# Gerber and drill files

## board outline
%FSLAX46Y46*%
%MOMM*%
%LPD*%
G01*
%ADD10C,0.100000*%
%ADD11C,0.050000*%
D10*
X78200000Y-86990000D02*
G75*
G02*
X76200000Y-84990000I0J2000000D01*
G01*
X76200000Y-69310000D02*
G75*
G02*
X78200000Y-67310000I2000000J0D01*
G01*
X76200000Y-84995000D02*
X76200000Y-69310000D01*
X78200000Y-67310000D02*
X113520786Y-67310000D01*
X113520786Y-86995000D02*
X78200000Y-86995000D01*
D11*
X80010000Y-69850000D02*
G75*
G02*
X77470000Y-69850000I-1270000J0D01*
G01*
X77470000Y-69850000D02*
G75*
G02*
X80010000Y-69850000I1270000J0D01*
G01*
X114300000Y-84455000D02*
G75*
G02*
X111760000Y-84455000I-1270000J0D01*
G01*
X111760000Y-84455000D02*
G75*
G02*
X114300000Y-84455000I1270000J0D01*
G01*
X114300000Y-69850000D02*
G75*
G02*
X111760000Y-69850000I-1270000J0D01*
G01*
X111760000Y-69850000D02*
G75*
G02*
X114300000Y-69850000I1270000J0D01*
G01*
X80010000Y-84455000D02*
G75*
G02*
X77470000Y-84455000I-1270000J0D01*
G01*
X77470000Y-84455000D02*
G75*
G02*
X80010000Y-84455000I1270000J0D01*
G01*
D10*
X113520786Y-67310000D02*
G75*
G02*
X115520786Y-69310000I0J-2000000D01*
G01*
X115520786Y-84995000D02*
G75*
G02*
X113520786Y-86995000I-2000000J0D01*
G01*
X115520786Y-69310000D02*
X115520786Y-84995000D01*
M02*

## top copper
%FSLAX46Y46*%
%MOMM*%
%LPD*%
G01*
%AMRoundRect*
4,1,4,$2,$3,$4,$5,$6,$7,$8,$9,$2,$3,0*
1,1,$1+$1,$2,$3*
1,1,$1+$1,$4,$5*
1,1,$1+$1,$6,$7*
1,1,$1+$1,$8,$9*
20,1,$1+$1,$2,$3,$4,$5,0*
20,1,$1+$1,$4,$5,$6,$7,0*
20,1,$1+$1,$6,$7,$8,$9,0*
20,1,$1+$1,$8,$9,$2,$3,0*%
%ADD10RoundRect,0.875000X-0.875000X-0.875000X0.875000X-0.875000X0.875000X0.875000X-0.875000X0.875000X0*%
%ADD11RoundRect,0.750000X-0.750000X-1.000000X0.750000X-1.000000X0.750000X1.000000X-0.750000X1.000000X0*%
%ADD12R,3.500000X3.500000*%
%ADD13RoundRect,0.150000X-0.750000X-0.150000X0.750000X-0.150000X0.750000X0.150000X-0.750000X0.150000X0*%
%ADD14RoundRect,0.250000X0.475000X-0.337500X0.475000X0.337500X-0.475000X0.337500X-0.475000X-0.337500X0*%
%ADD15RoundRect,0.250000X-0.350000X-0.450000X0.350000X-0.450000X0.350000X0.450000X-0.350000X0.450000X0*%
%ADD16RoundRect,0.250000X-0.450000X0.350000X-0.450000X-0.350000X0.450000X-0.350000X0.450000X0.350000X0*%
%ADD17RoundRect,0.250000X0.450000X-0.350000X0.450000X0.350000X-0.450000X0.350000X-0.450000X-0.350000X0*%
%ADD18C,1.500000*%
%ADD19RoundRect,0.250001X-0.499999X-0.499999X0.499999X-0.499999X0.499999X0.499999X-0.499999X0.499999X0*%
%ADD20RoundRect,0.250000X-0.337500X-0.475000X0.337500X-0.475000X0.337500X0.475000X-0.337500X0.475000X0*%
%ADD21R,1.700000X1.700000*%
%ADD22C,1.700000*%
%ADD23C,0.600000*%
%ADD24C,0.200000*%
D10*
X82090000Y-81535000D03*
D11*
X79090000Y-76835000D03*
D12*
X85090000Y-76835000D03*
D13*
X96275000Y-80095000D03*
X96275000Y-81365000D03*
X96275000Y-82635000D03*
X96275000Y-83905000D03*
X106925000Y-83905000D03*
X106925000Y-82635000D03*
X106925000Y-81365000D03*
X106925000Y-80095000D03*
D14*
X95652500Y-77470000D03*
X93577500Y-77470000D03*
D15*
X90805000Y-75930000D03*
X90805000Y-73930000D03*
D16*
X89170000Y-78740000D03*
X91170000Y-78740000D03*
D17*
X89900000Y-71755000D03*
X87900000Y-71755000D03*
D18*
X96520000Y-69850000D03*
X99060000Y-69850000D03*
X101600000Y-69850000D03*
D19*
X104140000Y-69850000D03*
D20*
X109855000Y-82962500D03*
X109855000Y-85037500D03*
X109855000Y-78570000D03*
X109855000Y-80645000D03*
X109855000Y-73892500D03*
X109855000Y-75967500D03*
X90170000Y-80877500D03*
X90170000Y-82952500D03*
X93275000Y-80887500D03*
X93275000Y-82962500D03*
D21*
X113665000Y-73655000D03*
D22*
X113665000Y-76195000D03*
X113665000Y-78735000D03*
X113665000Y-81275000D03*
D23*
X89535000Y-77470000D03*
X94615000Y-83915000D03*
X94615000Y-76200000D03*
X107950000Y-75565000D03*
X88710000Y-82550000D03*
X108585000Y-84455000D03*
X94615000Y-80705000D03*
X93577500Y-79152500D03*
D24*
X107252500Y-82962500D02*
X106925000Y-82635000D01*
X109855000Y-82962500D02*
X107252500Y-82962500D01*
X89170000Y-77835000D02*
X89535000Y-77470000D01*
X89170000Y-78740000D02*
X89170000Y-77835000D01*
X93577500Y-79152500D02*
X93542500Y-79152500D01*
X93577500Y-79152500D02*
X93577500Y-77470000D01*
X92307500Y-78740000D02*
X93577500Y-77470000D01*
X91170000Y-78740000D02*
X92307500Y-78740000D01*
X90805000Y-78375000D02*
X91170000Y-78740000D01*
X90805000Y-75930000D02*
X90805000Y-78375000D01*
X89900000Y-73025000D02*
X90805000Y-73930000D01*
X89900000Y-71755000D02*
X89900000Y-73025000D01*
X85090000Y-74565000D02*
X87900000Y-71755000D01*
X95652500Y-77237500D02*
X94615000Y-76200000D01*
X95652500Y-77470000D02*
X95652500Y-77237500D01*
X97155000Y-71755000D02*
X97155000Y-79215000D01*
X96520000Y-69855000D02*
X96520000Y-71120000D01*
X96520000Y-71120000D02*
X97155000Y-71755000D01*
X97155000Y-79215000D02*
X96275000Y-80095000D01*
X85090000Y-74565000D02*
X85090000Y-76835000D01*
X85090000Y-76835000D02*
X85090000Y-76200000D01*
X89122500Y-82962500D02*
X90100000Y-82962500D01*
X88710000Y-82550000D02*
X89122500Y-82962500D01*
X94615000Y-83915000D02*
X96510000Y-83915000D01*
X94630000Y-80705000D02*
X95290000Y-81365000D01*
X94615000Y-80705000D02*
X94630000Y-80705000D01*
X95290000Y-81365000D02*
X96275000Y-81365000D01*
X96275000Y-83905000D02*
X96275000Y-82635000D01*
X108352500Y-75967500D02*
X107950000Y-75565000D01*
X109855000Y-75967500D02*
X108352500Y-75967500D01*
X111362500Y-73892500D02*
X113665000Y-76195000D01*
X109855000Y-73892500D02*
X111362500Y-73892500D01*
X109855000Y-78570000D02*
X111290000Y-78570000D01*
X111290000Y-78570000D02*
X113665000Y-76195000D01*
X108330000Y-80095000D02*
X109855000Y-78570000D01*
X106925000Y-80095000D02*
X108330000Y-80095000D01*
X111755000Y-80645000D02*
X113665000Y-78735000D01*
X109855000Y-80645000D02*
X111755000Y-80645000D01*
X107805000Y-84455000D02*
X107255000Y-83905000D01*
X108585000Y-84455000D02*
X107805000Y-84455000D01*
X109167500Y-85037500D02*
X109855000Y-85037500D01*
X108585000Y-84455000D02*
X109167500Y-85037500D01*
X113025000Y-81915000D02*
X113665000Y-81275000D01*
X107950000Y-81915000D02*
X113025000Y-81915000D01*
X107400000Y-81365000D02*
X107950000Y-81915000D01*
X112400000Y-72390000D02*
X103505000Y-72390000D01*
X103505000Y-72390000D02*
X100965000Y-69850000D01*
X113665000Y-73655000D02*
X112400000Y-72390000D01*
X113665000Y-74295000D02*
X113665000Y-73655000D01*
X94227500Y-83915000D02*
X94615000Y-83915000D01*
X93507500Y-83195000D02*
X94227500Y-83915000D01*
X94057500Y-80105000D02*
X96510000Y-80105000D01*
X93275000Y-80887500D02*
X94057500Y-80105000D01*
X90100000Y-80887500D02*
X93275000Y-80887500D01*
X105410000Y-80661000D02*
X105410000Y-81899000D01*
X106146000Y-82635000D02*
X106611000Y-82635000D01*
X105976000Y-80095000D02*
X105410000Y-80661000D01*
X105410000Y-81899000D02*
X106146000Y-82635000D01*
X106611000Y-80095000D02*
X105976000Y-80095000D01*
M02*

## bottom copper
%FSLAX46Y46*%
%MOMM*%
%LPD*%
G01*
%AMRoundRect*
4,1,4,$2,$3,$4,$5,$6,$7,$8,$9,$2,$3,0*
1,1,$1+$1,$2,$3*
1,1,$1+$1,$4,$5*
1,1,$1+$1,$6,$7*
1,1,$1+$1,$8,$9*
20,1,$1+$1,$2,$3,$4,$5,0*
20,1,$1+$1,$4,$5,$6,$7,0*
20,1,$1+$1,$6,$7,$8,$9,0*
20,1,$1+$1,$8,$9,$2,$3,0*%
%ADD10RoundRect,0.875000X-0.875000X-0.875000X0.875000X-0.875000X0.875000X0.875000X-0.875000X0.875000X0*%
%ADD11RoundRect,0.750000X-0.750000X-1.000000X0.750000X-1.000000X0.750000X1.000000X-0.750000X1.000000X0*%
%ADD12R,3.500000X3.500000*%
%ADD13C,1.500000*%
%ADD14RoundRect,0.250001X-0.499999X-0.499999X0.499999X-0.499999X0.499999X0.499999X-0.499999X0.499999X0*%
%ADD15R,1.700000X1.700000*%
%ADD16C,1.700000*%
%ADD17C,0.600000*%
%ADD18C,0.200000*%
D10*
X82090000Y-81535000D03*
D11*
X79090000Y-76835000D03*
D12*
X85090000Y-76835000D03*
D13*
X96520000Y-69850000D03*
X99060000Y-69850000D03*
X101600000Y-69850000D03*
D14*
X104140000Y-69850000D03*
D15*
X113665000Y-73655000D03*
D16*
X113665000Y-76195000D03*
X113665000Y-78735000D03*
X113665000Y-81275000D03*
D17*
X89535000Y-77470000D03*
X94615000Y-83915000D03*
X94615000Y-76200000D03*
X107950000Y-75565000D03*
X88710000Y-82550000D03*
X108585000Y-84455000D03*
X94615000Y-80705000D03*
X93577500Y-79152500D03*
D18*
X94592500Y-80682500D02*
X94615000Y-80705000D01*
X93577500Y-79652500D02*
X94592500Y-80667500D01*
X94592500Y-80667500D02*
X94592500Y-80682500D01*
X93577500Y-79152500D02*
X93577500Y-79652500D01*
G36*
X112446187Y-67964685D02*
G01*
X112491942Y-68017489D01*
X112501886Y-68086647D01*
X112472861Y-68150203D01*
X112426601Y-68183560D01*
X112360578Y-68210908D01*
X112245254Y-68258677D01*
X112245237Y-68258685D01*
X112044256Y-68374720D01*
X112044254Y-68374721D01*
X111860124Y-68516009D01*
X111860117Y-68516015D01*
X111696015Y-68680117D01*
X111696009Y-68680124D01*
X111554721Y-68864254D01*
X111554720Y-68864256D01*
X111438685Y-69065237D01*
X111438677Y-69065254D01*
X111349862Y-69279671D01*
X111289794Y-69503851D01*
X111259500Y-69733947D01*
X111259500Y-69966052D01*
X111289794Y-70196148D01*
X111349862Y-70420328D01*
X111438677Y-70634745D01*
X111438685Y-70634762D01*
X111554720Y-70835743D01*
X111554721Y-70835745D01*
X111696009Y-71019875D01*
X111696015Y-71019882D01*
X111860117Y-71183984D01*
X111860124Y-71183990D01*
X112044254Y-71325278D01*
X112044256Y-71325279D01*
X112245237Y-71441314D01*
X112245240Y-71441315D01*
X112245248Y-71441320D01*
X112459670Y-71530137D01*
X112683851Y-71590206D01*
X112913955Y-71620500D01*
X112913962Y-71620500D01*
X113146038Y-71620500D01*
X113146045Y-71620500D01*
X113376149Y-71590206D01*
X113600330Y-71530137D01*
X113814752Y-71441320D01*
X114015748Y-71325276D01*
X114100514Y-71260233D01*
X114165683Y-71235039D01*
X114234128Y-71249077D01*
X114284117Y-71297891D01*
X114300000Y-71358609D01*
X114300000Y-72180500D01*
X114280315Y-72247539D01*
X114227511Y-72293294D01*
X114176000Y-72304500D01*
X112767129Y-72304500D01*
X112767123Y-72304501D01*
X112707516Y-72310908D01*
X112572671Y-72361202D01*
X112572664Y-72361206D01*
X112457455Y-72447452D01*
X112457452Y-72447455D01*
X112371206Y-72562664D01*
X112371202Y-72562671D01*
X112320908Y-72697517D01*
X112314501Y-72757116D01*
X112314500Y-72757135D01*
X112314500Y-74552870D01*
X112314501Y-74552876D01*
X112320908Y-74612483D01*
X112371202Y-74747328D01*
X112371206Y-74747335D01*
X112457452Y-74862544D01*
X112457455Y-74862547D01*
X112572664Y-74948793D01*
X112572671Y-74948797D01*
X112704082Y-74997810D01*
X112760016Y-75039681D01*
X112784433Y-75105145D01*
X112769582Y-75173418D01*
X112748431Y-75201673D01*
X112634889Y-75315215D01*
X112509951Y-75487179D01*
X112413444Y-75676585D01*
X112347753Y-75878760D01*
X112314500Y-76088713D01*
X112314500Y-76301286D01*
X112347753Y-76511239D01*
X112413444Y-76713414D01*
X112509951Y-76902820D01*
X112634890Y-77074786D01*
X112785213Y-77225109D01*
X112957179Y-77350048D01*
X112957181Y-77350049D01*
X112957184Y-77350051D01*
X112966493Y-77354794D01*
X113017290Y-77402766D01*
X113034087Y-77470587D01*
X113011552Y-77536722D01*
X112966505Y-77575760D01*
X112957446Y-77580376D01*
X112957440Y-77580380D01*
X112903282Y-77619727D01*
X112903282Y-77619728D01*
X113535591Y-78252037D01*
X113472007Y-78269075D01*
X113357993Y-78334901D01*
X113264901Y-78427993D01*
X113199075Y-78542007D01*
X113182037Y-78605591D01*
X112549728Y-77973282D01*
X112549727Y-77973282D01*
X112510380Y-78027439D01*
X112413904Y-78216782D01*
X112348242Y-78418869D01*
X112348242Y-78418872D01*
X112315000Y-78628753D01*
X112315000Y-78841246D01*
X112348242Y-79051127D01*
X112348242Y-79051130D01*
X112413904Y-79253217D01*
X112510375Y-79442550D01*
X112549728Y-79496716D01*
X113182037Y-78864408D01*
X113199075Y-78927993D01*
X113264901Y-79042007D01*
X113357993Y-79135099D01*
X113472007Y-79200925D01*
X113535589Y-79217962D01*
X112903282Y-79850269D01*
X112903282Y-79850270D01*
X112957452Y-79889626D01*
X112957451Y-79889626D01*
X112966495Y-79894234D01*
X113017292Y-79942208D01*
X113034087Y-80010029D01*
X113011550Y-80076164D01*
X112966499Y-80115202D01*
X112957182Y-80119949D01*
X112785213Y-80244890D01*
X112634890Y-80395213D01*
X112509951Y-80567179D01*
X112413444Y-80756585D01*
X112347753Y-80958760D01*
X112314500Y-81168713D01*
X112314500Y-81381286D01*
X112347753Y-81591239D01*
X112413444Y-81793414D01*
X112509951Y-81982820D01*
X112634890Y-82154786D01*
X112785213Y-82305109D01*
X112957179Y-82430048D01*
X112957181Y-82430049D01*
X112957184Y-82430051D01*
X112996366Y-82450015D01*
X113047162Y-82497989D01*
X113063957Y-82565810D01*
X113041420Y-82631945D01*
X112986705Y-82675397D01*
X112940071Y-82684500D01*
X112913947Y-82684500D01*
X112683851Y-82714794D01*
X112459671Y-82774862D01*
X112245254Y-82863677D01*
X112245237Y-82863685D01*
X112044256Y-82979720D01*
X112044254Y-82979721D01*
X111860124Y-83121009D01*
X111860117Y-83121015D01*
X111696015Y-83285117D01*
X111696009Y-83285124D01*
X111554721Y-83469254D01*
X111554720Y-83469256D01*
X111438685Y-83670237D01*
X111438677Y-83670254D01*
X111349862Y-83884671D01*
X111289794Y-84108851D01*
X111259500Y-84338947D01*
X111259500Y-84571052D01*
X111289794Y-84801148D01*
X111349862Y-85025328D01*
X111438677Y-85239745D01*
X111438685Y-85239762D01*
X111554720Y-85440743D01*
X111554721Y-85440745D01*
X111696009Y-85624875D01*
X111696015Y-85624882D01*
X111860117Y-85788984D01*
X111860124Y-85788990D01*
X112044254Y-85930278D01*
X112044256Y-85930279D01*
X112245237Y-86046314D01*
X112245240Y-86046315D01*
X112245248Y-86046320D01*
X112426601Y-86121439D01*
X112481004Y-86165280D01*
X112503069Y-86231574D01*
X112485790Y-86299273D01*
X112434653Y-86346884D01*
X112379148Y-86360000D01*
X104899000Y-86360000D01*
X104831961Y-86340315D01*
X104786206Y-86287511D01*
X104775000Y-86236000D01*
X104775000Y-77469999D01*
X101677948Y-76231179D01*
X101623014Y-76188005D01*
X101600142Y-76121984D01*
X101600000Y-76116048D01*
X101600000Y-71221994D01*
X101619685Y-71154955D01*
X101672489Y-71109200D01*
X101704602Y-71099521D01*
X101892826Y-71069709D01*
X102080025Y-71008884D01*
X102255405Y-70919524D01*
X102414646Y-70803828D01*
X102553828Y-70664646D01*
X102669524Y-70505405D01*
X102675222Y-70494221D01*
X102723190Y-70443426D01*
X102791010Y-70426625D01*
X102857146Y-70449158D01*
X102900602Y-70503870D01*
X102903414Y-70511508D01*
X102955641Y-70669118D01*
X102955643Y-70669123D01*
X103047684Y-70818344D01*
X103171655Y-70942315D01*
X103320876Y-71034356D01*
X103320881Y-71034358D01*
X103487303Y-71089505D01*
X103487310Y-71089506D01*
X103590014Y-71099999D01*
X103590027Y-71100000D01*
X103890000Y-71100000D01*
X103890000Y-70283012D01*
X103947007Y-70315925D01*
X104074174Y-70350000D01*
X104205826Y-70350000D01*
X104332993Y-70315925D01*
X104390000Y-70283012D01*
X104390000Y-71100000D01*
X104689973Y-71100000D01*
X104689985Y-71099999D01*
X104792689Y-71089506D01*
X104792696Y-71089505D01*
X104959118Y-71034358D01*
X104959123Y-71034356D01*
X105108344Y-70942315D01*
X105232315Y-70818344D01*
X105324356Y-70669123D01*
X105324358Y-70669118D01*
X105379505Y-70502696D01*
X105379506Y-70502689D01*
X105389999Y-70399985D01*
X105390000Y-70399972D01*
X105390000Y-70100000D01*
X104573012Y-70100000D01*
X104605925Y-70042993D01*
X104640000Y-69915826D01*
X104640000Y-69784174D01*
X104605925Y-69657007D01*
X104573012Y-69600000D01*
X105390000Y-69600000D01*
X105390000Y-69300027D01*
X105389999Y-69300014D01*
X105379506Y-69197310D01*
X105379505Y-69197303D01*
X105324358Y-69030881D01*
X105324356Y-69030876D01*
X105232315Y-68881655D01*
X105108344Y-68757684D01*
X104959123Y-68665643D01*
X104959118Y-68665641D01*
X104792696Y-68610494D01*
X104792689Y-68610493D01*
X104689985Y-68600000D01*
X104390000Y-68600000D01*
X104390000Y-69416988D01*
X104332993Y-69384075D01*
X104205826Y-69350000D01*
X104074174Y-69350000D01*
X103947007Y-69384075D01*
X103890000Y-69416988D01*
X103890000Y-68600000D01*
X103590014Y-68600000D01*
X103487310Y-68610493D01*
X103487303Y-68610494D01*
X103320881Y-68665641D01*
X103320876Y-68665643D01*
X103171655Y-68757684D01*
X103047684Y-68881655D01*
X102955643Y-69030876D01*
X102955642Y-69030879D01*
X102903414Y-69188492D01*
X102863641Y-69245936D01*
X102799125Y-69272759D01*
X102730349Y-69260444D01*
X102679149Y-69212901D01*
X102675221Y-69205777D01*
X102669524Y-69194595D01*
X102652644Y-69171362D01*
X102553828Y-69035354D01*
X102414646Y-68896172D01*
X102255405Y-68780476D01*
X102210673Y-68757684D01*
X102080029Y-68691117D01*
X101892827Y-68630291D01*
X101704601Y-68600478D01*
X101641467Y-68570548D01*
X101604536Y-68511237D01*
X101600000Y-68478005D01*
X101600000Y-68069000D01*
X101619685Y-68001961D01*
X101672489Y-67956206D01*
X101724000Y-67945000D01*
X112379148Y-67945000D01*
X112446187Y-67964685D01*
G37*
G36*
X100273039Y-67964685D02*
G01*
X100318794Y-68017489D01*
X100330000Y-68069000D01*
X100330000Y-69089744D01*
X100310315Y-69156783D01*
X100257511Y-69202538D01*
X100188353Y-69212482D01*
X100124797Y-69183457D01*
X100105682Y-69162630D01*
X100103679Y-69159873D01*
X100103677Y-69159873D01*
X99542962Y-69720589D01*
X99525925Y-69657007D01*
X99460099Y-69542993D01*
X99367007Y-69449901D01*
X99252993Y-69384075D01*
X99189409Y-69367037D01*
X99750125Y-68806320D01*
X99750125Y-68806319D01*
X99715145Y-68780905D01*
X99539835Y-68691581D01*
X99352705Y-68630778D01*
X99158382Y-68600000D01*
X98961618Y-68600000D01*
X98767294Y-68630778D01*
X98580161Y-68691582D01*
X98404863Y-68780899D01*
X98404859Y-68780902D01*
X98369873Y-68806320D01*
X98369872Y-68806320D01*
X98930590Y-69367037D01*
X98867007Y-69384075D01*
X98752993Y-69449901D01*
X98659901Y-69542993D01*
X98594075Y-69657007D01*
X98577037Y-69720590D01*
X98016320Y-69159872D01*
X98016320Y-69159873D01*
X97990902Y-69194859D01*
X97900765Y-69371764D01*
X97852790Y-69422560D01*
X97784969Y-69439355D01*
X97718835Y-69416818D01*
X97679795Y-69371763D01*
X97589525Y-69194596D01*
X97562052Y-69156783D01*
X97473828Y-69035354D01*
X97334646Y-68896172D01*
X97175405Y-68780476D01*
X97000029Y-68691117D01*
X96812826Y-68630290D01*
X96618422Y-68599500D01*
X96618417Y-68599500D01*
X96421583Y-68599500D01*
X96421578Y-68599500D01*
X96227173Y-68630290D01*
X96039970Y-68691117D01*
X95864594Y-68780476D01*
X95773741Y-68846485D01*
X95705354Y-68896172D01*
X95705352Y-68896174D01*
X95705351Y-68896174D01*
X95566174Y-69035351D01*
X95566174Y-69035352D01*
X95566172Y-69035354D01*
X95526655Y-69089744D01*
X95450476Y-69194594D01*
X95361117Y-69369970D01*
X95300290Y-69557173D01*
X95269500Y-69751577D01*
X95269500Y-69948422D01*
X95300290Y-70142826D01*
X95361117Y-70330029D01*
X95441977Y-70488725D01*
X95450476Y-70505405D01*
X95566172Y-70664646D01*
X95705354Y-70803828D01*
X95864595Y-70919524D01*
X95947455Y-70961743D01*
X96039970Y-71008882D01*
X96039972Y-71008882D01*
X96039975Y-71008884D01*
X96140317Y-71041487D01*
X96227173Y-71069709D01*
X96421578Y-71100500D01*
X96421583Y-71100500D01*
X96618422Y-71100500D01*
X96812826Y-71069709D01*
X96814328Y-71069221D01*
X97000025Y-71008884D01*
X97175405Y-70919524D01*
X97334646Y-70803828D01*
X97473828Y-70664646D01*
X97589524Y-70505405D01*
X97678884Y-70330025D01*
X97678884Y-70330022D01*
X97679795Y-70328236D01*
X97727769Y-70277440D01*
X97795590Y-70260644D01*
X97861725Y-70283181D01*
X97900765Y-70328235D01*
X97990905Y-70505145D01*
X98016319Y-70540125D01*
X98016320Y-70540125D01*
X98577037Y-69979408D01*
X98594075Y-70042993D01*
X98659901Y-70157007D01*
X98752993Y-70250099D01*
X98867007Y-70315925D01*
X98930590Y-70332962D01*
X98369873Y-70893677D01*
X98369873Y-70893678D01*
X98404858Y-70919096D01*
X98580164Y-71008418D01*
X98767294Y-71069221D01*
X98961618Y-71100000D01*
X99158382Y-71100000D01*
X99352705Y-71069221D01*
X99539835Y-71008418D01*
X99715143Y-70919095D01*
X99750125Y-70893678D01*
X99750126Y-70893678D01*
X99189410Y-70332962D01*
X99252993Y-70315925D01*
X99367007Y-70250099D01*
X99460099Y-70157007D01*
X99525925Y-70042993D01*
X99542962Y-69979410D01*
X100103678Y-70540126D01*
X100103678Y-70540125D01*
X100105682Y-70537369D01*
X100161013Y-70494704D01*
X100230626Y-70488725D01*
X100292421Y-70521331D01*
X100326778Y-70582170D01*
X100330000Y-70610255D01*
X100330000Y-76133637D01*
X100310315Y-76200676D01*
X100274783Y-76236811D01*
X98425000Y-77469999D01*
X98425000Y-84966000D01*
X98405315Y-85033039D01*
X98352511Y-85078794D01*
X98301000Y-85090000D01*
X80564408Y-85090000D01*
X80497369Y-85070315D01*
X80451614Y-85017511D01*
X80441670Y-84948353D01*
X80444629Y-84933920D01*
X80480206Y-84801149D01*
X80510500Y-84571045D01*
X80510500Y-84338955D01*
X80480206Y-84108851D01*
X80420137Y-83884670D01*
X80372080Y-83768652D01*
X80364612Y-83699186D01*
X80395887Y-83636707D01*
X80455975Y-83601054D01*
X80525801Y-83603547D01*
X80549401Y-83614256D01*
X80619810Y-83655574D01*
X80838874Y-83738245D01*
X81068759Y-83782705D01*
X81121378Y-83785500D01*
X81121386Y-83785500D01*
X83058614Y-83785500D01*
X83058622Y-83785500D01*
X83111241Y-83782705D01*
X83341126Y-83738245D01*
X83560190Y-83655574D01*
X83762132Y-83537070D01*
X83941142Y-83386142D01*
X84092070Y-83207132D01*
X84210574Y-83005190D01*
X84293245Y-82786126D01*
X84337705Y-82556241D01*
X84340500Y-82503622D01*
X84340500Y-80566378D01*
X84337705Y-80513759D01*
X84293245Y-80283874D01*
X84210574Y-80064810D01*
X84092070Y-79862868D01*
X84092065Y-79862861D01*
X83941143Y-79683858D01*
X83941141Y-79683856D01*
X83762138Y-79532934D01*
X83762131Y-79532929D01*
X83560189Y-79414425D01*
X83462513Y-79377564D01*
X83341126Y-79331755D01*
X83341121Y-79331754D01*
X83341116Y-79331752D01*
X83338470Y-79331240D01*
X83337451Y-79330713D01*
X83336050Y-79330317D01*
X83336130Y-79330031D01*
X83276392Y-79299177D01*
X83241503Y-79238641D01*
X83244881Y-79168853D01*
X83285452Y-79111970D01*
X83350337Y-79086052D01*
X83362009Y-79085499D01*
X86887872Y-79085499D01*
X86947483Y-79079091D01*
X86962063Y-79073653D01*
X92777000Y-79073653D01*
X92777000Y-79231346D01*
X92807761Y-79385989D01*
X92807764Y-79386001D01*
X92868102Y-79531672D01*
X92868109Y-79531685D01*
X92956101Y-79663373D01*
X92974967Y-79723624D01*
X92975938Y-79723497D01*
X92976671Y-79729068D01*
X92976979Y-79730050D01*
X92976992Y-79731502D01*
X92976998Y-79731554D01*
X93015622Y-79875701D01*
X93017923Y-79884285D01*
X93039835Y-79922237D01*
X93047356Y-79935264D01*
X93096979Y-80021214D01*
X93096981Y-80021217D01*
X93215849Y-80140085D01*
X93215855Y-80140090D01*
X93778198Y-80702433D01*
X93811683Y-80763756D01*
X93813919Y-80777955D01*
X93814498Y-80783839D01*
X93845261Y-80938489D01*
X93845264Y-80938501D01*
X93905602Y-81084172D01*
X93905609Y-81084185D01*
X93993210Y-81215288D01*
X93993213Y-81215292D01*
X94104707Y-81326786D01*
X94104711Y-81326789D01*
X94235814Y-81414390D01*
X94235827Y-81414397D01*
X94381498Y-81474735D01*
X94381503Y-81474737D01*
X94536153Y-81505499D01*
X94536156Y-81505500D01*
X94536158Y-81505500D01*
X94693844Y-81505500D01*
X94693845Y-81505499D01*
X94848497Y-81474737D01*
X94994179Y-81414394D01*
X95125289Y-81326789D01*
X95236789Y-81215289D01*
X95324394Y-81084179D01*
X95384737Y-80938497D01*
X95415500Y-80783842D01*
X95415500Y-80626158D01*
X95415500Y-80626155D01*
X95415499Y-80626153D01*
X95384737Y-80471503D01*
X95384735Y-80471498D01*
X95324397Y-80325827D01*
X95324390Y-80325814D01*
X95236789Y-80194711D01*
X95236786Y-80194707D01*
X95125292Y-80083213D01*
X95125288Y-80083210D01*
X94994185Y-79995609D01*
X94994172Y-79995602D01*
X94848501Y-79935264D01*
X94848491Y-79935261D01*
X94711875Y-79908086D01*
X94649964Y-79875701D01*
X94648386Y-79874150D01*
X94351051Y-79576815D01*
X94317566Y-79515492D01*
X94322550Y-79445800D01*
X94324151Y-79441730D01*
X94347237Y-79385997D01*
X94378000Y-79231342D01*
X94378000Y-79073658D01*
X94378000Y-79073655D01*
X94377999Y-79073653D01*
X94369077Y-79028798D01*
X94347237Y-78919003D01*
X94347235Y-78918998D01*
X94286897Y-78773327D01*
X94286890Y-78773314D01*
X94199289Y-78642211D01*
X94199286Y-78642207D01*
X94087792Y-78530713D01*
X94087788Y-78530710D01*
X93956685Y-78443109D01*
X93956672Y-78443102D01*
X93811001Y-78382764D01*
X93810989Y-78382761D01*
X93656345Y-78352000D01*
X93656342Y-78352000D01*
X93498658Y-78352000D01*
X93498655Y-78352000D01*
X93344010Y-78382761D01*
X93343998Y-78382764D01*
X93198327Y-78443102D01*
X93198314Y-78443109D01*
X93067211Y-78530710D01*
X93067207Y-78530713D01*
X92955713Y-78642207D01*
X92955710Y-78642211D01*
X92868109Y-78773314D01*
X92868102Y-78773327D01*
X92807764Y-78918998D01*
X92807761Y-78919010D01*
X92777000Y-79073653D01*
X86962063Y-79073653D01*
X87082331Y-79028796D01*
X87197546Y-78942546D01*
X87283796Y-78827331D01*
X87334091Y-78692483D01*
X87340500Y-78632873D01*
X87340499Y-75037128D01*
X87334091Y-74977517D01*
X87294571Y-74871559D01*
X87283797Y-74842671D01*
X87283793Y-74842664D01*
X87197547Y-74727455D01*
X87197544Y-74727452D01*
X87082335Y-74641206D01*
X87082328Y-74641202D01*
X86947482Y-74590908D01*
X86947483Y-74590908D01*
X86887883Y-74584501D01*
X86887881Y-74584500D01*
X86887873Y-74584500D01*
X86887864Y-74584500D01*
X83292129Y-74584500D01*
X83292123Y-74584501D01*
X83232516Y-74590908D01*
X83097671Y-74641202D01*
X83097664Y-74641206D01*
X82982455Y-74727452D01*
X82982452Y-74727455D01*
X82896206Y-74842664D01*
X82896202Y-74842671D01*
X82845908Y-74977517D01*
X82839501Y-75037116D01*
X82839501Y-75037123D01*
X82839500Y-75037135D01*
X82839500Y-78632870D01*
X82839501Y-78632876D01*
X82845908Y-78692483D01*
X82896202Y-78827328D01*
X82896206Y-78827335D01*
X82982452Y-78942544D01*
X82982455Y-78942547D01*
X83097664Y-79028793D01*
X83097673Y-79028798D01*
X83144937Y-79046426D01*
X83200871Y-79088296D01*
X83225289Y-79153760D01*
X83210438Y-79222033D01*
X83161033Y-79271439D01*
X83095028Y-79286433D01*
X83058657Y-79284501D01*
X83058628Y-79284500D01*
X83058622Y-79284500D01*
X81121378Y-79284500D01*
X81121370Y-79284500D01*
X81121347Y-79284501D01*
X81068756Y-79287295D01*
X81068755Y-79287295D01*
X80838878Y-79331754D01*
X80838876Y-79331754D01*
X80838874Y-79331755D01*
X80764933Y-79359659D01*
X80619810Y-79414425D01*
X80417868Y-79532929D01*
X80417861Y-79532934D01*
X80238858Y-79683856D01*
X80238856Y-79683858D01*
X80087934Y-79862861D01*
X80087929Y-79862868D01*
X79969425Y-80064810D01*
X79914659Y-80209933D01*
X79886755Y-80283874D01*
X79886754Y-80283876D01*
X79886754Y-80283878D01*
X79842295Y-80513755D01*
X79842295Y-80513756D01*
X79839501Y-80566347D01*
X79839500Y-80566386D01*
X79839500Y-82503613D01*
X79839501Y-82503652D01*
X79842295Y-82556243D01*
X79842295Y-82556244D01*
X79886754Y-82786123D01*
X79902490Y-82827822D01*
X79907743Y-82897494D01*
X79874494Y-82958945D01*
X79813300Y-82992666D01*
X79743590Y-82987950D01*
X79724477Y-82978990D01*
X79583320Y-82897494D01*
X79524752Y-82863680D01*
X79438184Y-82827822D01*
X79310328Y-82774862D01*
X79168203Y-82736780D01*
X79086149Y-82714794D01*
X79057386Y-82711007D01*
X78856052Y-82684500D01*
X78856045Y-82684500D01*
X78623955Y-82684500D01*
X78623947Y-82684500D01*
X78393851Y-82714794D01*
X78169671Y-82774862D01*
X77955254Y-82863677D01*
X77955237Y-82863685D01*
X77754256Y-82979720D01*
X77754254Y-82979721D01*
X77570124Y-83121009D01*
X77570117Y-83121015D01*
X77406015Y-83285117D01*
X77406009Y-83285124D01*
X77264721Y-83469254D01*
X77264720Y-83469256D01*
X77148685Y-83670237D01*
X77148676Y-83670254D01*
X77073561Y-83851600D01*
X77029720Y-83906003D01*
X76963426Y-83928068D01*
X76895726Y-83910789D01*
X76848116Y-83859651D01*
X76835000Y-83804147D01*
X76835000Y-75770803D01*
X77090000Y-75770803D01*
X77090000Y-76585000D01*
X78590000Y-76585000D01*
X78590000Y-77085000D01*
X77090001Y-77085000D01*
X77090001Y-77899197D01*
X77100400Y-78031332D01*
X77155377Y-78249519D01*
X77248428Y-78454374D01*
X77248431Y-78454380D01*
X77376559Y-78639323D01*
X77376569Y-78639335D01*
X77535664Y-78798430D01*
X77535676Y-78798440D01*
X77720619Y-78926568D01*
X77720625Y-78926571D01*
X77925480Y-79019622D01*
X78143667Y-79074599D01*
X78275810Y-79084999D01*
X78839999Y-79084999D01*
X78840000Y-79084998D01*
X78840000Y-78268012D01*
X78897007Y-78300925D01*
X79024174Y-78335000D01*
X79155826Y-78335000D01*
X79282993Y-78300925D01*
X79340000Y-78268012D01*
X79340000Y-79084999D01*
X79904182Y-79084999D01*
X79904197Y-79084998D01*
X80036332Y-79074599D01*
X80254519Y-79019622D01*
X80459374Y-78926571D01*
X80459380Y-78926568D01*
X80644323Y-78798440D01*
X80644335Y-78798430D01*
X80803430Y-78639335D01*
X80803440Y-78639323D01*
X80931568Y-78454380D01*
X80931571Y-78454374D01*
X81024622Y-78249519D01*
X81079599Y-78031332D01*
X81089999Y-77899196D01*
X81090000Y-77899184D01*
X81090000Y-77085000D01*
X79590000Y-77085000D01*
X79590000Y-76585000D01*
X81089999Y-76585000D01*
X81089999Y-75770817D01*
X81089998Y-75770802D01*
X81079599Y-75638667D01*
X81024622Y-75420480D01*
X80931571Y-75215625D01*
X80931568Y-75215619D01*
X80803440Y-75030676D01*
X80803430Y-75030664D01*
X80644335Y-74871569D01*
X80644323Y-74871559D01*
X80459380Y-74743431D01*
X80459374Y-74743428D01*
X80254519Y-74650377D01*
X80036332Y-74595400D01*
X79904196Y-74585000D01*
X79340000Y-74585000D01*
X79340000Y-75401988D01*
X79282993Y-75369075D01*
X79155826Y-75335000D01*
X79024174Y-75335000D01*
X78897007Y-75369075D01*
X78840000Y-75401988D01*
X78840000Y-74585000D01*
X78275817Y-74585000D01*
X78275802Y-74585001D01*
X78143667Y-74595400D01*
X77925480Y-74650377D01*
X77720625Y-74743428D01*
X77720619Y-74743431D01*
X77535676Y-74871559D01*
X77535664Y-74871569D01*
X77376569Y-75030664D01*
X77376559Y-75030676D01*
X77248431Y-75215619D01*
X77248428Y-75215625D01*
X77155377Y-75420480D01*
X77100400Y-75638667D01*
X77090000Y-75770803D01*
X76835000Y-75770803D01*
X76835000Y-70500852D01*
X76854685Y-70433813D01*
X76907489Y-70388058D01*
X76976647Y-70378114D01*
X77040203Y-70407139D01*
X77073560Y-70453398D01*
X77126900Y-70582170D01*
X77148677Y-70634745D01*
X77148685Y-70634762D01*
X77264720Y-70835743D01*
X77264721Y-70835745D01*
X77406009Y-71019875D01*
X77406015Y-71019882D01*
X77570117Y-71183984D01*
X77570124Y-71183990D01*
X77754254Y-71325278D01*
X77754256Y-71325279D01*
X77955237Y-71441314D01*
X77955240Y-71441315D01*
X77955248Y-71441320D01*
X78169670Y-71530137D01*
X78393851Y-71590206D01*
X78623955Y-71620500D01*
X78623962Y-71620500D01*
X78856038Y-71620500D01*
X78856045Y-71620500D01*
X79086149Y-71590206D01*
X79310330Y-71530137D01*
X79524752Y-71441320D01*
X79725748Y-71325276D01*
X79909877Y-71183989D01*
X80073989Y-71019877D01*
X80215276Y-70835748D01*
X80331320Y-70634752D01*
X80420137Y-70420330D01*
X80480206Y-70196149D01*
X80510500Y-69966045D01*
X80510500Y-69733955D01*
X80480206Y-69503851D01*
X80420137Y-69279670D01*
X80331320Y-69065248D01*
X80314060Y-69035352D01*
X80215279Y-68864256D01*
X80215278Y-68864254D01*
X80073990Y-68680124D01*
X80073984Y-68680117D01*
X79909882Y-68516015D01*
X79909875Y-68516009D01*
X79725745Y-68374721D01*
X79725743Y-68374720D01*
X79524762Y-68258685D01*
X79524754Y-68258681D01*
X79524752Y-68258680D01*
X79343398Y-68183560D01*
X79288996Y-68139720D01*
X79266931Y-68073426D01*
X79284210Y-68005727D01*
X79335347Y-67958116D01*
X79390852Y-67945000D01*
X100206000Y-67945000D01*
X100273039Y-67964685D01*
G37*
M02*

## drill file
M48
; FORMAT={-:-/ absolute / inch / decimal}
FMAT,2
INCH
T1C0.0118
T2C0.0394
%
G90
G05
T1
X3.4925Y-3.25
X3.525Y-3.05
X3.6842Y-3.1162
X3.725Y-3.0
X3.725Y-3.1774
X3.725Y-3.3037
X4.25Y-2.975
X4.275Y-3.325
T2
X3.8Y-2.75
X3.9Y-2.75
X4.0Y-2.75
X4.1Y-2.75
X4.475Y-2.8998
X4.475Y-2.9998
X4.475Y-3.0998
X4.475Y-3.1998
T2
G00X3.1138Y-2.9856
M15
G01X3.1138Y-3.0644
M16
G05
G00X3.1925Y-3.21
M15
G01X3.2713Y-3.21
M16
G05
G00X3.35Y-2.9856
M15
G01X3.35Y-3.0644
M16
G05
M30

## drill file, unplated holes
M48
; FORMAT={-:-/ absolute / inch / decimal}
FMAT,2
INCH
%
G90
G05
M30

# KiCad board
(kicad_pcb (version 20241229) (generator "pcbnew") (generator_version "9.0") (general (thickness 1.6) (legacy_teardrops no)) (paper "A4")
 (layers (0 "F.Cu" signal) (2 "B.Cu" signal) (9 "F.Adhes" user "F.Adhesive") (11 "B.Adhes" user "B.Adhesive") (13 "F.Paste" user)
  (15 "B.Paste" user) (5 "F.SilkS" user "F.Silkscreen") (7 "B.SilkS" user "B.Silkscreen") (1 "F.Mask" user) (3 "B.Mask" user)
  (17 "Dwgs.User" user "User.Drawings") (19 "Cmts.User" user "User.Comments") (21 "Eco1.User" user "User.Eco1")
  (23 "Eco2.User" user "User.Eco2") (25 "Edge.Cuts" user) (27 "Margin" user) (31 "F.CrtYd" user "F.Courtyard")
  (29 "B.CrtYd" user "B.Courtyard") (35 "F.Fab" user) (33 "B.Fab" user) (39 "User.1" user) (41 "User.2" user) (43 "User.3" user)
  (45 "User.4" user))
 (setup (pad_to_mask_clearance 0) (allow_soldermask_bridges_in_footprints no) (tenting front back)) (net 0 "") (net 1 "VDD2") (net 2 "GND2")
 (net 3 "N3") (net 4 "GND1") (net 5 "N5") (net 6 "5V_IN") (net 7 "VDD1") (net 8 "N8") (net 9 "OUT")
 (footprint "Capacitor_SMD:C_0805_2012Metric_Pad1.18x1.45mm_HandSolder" (layer "F.Cu") (at 109.855 84 -90)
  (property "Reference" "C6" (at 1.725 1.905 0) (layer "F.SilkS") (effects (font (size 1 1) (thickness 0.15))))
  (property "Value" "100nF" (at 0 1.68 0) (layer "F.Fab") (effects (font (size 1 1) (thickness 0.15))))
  (pad "1" smd roundrect (at -1.0375 0) (size 1.175 1.45) (layers "F.Cu" "F.Mask" "F.Paste") (roundrect_rratio 0.212766) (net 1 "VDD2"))
  (pad "2" smd roundrect (at 1.0375 0) (size 1.175 1.45) (layers "F.Cu" "F.Mask" "F.Paste") (roundrect_rratio 0.212766) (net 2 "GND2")))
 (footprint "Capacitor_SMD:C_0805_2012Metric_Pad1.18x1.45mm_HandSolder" (layer "F.Cu") (at 109.855 79.6075 -90)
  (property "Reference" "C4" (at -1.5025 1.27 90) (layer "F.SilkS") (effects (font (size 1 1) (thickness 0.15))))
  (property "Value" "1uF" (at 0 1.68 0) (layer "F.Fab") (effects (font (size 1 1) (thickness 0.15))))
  (pad "1" smd roundrect (at -1.0375 0) (size 1.175 1.45) (layers "F.Cu" "F.Mask" "F.Paste") (roundrect_rratio 0.212766) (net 1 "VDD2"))
  (pad "2" smd roundrect (at 1.0375 0) (size 1.175 1.45) (layers "F.Cu" "F.Mask" "F.Paste") (roundrect_rratio 0.212766) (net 2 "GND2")))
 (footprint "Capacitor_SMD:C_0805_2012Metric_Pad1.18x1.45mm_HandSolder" (layer "F.Cu") (at 94.615 77.47)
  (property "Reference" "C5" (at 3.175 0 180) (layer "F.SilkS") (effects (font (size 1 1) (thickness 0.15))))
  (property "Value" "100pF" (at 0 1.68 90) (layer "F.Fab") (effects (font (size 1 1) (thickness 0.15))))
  (pad "1" smd roundrect (at -1.0375 0 90) (size 1.175 1.45) (layers "F.Cu" "F.Mask" "F.Paste") (roundrect_rratio 0.212766) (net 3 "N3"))
  (pad "2" smd roundrect (at 1.0375 0 90) (size 1.175 1.45) (layers "F.Cu" "F.Mask" "F.Paste") (roundrect_rratio 0.212766) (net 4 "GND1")))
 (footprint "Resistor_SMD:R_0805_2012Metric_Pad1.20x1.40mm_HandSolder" (layer "F.Cu") (at 90.805 74.93 -90)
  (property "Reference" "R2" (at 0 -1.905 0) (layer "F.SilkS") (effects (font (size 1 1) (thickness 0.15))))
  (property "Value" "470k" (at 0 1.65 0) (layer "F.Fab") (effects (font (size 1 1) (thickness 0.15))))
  (pad "1" smd roundrect (at -1 0) (size 1.2 1.4) (layers "F.Cu" "F.Mask" "F.Paste") (roundrect_rratio 0.208333) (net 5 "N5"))
  (pad "2" smd roundrect (at 1 0) (size 1.2 1.4) (layers "F.Cu" "F.Mask" "F.Paste") (roundrect_rratio 0.208333) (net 3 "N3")))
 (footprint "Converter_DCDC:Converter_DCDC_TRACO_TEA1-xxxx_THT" (layer "F.Cu") (at 104.14 69.85 -90)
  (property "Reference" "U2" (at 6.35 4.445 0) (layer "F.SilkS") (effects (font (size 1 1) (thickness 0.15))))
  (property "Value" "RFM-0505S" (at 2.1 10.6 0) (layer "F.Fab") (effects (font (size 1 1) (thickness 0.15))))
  (pad "1" thru_hole roundrect (at 0 0) (size 1.5 1.5) (drill 1) (layers "*.Cu" "*.Mask") (remove_unused_layers no)
   (roundrect_rratio 0.166667) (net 2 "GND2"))
  (pad "2" thru_hole circle (at 0 2.54) (size 1.5 1.5) (drill 1) (layers "*.Cu" "*.Mask") (remove_unused_layers no) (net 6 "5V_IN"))
  (pad "3" thru_hole circle (at 0 5.08) (size 1.5 1.5) (drill 1) (layers "*.Cu" "*.Mask") (remove_unused_layers no) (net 4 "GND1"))
  (pad "4" thru_hole circle (at 0 7.62) (size 1.5 1.5) (drill 1) (layers "*.Cu" "*.Mask") (remove_unused_layers no) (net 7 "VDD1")))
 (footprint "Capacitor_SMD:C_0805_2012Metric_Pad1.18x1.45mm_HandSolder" (layer "F.Cu") (at 109.855 74.93 -90)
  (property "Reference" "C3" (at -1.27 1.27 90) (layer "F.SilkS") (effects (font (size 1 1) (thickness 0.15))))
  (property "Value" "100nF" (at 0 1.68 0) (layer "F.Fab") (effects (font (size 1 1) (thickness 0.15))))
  (pad "1" smd roundrect (at -1.0375 0) (size 1.175 1.45) (layers "F.Cu" "F.Mask" "F.Paste") (roundrect_rratio 0.212766) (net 1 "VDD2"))
  (pad "2" smd roundrect (at 1.0375 0) (size 1.175 1.45) (layers "F.Cu" "F.Mask" "F.Paste") (roundrect_rratio 0.212766) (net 2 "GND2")))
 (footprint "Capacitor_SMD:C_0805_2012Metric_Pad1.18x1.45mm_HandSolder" (layer "F.Cu") (at 90.17 81.915 -90)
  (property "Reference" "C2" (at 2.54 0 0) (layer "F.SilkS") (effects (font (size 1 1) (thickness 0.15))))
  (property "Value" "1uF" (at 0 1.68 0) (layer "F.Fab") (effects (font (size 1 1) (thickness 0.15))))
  (pad "1" smd roundrect (at -1.0375 0) (size 1.175 1.45) (layers "F.Cu" "F.Mask" "F.Paste") (roundrect_rratio 0.212766) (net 7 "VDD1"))
  (pad "2" smd roundrect (at 1.0375 0) (size 1.175 1.45) (layers "F.Cu" "F.Mask" "F.Paste") (roundrect_rratio 0.212766) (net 4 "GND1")))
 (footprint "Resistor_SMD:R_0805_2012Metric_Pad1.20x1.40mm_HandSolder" (layer "F.Cu") (at 90.17 78.74 180)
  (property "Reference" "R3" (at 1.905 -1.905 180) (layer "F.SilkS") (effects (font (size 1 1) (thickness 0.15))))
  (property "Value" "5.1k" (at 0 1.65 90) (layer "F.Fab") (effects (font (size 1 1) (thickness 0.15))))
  (pad "1" smd roundrect (at -1 0 270) (size 1.2 1.4) (layers "F.Cu" "F.Mask" "F.Paste") (roundrect_rratio 0.208333) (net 3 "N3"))
  (pad "2" smd roundrect (at 1 0 270) (size 1.2 1.4) (layers "F.Cu" "F.Mask" "F.Paste") (roundrect_rratio 0.208333) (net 4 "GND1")))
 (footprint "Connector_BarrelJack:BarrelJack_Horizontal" (layer "F.Cu") (at 85.09 76.835)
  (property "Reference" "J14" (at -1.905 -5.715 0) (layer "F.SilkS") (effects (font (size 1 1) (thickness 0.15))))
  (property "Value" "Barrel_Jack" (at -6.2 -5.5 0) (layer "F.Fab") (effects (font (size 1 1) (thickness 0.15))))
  (pad "1" thru_hole rect (at 0 0) (size 3.5 3.5) (drill oval 1 3) (layers "*.Cu" "*.Mask") (remove_unused_layers no) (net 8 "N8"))
  (pad "2" thru_hole roundrect (at -6 0) (size 3 3.5) (drill oval 1 3) (layers "*.Cu" "*.Mask") (remove_unused_layers no)
   (roundrect_rratio 0.25) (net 4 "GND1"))
  (pad "3" thru_hole roundrect (at -3 4.7) (size 3.5 3.5) (drill oval 3 1) (layers "*.Cu" "*.Mask") (remove_unused_layers no)
   (roundrect_rratio 0.25)))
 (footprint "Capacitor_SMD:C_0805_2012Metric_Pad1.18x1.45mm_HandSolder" (layer "F.Cu") (at 93.275 81.925 -90)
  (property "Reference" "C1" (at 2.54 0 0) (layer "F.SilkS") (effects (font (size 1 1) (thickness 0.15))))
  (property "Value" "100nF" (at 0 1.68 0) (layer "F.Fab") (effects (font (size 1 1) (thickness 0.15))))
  (pad "1" smd roundrect (at -1.0375 0) (size 1.175 1.45) (layers "F.Cu" "F.Mask" "F.Paste") (roundrect_rratio 0.212766) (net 7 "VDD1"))
  (pad "2" smd roundrect (at 1.0375 0) (size 1.175 1.45) (layers "F.Cu" "F.Mask" "F.Paste") (roundrect_rratio 0.212766) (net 4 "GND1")))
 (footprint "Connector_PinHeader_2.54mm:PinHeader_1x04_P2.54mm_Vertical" (layer "F.Cu") (at 113.665 73.655)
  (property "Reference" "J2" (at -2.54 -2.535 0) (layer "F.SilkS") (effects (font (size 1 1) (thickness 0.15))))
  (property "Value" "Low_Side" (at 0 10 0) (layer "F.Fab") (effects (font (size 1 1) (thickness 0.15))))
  (pad "1" thru_hole rect (at 0 0) (size 1.7 1.7) (drill 1) (layers "*.Cu" "*.Mask") (remove_unused_layers no) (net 6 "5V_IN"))
  (pad "2" thru_hole circle (at 0 2.54) (size 1.7 1.7) (drill 1) (layers "*.Cu" "*.Mask") (remove_unused_layers no) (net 1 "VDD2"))
  (pad "3" thru_hole circle (at 0 5.08) (size 1.7 1.7) (drill 1) (layers "*.Cu" "*.Mask") (remove_unused_layers no) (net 2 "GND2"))
  (pad "4" thru_hole circle (at 0 7.62) (size 1.7 1.7) (drill 1) (layers "*.Cu" "*.Mask") (remove_unused_layers no) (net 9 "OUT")))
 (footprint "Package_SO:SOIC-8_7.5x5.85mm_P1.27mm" (layer "F.Cu") (at 101.6 82)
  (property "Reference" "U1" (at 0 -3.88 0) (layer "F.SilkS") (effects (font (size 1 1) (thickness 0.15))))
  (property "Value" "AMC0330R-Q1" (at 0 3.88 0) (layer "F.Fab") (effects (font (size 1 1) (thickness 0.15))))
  (pad "1" smd roundrect (at -5.325 -1.905) (size 1.8 0.6) (layers "F.Cu" "F.Mask" "F.Paste") (roundrect_rratio 0.25) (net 7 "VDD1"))
  (pad "2" smd roundrect (at -5.325 -0.635) (size 1.8 0.6) (layers "F.Cu" "F.Mask" "F.Paste") (roundrect_rratio 0.25) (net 3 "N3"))
  (pad "3" smd roundrect (at -5.325 0.635) (size 1.8 0.6) (layers "F.Cu" "F.Mask" "F.Paste") (roundrect_rratio 0.25) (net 4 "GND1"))
  (pad "4" smd roundrect (at -5.325 1.905) (size 1.8 0.6) (layers "F.Cu" "F.Mask" "F.Paste") (roundrect_rratio 0.25) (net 4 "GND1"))
  (pad "5" smd roundrect (at 5.325 1.905) (size 1.8 0.6) (layers "F.Cu" "F.Mask" "F.Paste") (roundrect_rratio 0.25) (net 2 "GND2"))
  (pad "6" smd roundrect (at 5.325 0.635) (size 1.8 0.6) (layers "F.Cu" "F.Mask" "F.Paste") (roundrect_rratio 0.25) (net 1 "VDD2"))
  (pad "7" smd roundrect (at 5.325 -0.635) (size 1.8 0.6) (layers "F.Cu" "F.Mask" "F.Paste") (roundrect_rratio 0.25) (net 9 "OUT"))
  (pad "8" smd roundrect (at 5.325 -1.905) (size 1.8 0.6) (layers "F.Cu" "F.Mask" "F.Paste") (roundrect_rratio 0.25) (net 1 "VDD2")))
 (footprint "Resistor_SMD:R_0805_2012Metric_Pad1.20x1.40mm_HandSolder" (layer "F.Cu") (at 88.9 71.755)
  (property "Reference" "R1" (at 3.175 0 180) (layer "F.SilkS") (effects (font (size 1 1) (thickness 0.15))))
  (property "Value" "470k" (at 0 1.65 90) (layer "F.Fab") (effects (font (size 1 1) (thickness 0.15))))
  (pad "1" smd roundrect (at -1 0 90) (size 1.2 1.4) (layers "F.Cu" "F.Mask" "F.Paste") (roundrect_rratio 0.208333) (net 8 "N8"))
  (pad "2" smd roundrect (at 1 0 90) (size 1.2 1.4) (layers "F.Cu" "F.Mask" "F.Paste") (roundrect_rratio 0.208333) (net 5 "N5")))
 (gr_arc (start 76.2 69.31) (mid 76.785786 67.895786) (end 78.2 67.31) (stroke (width 0.1) (type default)) (layer "Edge.Cuts"))
 (gr_line (start 115.520786 69.31) (end 115.520786 84.995) (stroke (width 0.1) (type default)) (layer "Edge.Cuts"))
 (gr_arc (start 115.520786 84.995) (mid 114.935 86.409214) (end 113.520786 86.995) (stroke (width 0.1) (type default)) (layer "Edge.Cuts"))
 (gr_line (start 78.2 67.31) (end 113.520786 67.31) (stroke (width 0.1) (type default)) (layer "Edge.Cuts"))
 (gr_circle (center 78.74 84.455) (end 78.74 83.185) (stroke (width 0.05) (type default)) (fill no) (layer "Edge.Cuts"))
 (gr_arc (start 78.2 86.99) (mid 76.785786 86.404214) (end 76.2 84.99) (stroke (width 0.1) (type default)) (layer "Edge.Cuts"))
 (gr_arc (start 113.520786 67.31) (mid 114.935 67.895786) (end 115.520786 69.31) (stroke (width 0.1) (type default)) (layer "Edge.Cuts"))
 (gr_line (start 76.2 84.995) (end 76.2 69.31) (stroke (width 0.1) (type default)) (layer "Edge.Cuts"))
 (gr_circle (center 113.03 69.85) (end 113.03 68.58) (stroke (width 0.05) (type default)) (fill no) (layer "Edge.Cuts"))
 (gr_circle (center 78.74 69.85) (end 78.74 68.58) (stroke (width 0.05) (type default)) (fill no) (layer "Edge.Cuts"))
 (gr_circle (center 113.03 84.455) (end 113.03 83.185) (stroke (width 0.05) (type default)) (fill no) (layer "Edge.Cuts"))
 (gr_line (start 113.520786 86.995) (end 78.2 86.995) (stroke (width 0.1) (type default)) (layer "Edge.Cuts"))
 (segment (start 89.17 78.74) (end 89.17 77.835) (width 0.2) (layer "F.Cu") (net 4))
 (segment (start 95.6525 77.47) (end 95.6525 77.2375) (width 0.2) (layer "F.Cu") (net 4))
 (segment (start 89.1225 82.9625) (end 90.1 82.9625) (width 0.2) (layer "F.Cu") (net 4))
 (segment (start 94.2275 83.915) (end 94.615 83.915) (width 0.2) (layer "F.Cu") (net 4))
 (segment (start 95.6525 77.2375) (end 94.615 76.2) (width 0.2) (layer "F.Cu") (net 4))
 (segment (start 94.615 83.915) (end 96.51 83.915) (width 0.2) (layer "F.Cu") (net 4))
 (segment (start 93.5075 83.195) (end 94.2275 83.915) (width 0.2) (layer "F.Cu") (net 4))
 (segment (start 96.275 83.905) (end 96.275 82.635) (width 0.2) (layer "F.Cu") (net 4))
 (segment (start 89.17 77.835) (end 89.535 77.47) (width 0.2) (layer "F.Cu") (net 4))
 (segment (start 88.71 82.55) (end 89.1225 82.9625) (width 0.2) (layer "F.Cu") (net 4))
 (via (at 94.615 76.2) (size 0.6) (drill 0.3) (layers "F.Cu" "B.Cu") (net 4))
 (via (at 94.615 83.915) (size 0.6) (drill 0.3) (layers "F.Cu" "B.Cu") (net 4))
 (via (at 89.535 77.47) (size 0.6) (drill 0.3) (layers "F.Cu" "B.Cu") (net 4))
 (via (at 88.71 82.55) (size 0.6) (drill 0.3) (layers "F.Cu" "B.Cu") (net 4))
 (segment (start 96.52 69.855) (end 96.52 71.12) (width 0.2) (layer "F.Cu") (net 7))
 (segment (start 90.1 80.8875) (end 93.275 80.8875) (width 0.2) (layer "F.Cu") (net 7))
 (segment (start 94.0575 80.105) (end 96.51 80.105) (width 0.2) (layer "F.Cu") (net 7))
 (segment (start 96.52 71.12) (end 97.155 71.755) (width 0.2) (layer "F.Cu") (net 7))
 (segment (start 97.155 71.755) (end 97.155 79.215) (width 0.2) (layer "F.Cu") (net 7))
 (segment (start 93.275 80.8875) (end 94.0575 80.105) (width 0.2) (layer "F.Cu") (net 7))
 (segment (start 97.155 79.215) (end 96.275 80.095) (width 0.2) (layer "F.Cu") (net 7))
 (segment (start 108.585 84.455) (end 107.805 84.455) (width 0.2) (layer "F.Cu") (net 2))
 (segment (start 109.855 80.645) (end 111.755 80.645) (width 0.2) (layer "F.Cu") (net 2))
 (segment (start 109.1675 85.0375) (end 109.855 85.0375) (width 0.2) (layer "F.Cu") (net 2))
 (segment (start 111.755 80.645) (end 113.665 78.735) (width 0.2) (layer "F.Cu") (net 2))
 (segment (start 108.3525 75.9675) (end 107.95 75.565) (width 0.2) (layer "F.Cu") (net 2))
 (segment (start 107.805 84.455) (end 107.255 83.905) (width 0.2) (layer "F.Cu") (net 2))
 (segment (start 108.585 84.455) (end 109.1675 85.0375) (width 0.2) (layer "F.Cu") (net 2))
 (segment (start 109.855 75.9675) (end 108.3525 75.9675) (width 0.2) (layer "F.Cu") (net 2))
 (via (at 108.585 84.455) (size 0.6) (drill 0.3) (layers "F.Cu" "B.Cu") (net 2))
 (via (at 107.95 75.565) (size 0.6) (drill 0.3) (layers "F.Cu" "B.Cu") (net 2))
 (segment (start 106.146 82.635) (end 106.611 82.635) (width 0.2) (layer "F.Cu") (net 1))
 (segment (start 111.3625 73.8925) (end 113.665 76.195) (width 0.2) (layer "F.Cu") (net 1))
 (segment (start 108.33 80.095) (end 109.855 78.57) (width 0.2) (layer "F.Cu") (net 1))
 (segment (start 107.2525 82.9625) (end 106.925 82.635) (width 0.2) (layer "F.Cu") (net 1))
 (segment (start 109.855 78.57) (end 111.29 78.57) (width 0.2) (layer "F.Cu") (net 1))
 (segment (start 109.855 73.8925) (end 111.3625 73.8925) (width 0.2) (layer "F.Cu") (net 1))
 (segment (start 111.29 78.57) (end 113.665 76.195) (width 0.2) (layer "F.Cu") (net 1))
 (segment (start 105.976 80.095) (end 105.41 80.661) (width 0.2) (layer "F.Cu") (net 1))
 (segment (start 105.41 81.899) (end 106.146 82.635) (width 0.2) (layer "F.Cu") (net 1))
 (segment (start 106.611 80.095) (end 105.976 80.095) (width 0.2) (layer "F.Cu") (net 1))
 (segment (start 106.925 80.095) (end 108.33 80.095) (width 0.2) (layer "F.Cu") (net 1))
 (segment (start 105.41 80.661) (end 105.41 81.899) (width 0.2) (layer "F.Cu") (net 1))
 (segment (start 109.855 82.9625) (end 107.2525 82.9625) (width 0.2) (layer "F.Cu") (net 1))
 (segment (start 92.3075 78.74) (end 93.5775 77.47) (width 0.2) (layer "F.Cu") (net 3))
 (segment (start 91.17 78.74) (end 92.3075 78.74) (width 0.2) (layer "F.Cu") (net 3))
 (segment (start 94.63 80.705) (end 95.29 81.365) (width 0.2) (layer "F.Cu") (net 3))
 (segment (start 93.5775 79.1525) (end 93.5425 79.1525) (width 0.2) (layer "F.Cu") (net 3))
 (segment (start 90.805 75.93) (end 90.805 78.375) (width 0.2) (layer "F.Cu") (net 3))
 (segment (start 93.5775 79.1525) (end 93.5775 77.47) (width 0.2) (layer "F.Cu") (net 3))
 (segment (start 94.615 80.705) (end 94.63 80.705) (width 0.2) (layer "F.Cu") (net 3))
 (segment (start 95.29 81.365) (end 96.275 81.365) (width 0.2) (layer "F.Cu") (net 3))
 (segment (start 90.805 78.375) (end 91.17 78.74) (width 0.2) (layer "F.Cu") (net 3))
 (via (at 93.5775 79.1525) (size 0.6) (drill 0.3) (layers "F.Cu" "B.Cu") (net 3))
 (via (at 94.615 80.705) (size 0.6) (drill 0.3) (layers "F.Cu" "B.Cu") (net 3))
 (segment (start 93.5775 79.1525) (end 93.5775 79.6525) (width 0.2) (layer "B.Cu") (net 3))
 (segment (start 94.5925 80.6675) (end 94.5925 80.6825) (width 0.2) (layer "B.Cu") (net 3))
 (segment (start 94.5925 80.6825) (end 94.615 80.705) (width 0.2) (layer "B.Cu") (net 3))
 (segment (start 93.5775 79.6525) (end 94.5925 80.6675) (width 0.2) (layer "B.Cu") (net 3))
 (segment (start 107.95 81.915) (end 113.025 81.915) (width 0.2) (layer "F.Cu") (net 9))
 (segment (start 113.025 81.915) (end 113.665 81.275) (width 0.2) (layer "F.Cu") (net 9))
 (segment (start 107.4 81.365) (end 107.95 81.915) (width 0.2) (layer "F.Cu") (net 9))
 (segment (start 112.4 72.39) (end 103.505 72.39) (width 0.2) (layer "F.Cu") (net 6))
 (segment (start 103.505 72.39) (end 100.965 69.85) (width 0.2) (layer "F.Cu") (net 6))
 (segment (start 113.665 74.295) (end 113.665 73.655) (width 0.2) (layer "F.Cu") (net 6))
 (segment (start 113.665 73.655) (end 112.4 72.39) (width 0.2) (layer "F.Cu") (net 6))
 (segment (start 89.9 71.755) (end 89.9 73.025) (width 0.2) (layer "F.Cu") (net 5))
 (segment (start 89.9 73.025) (end 90.805 73.93) (width 0.2) (layer "F.Cu") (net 5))
 (segment (start 85.09 74.565) (end 87.9 71.755) (width 0.2) (layer "F.Cu") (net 8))
 (segment (start 85.09 74.565) (end 85.09 76.835) (width 0.2) (layer "F.Cu") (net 8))
 (segment (start 85.09 76.835) (end 85.09 76.2) (width 0.2) (layer "F.Cu") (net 8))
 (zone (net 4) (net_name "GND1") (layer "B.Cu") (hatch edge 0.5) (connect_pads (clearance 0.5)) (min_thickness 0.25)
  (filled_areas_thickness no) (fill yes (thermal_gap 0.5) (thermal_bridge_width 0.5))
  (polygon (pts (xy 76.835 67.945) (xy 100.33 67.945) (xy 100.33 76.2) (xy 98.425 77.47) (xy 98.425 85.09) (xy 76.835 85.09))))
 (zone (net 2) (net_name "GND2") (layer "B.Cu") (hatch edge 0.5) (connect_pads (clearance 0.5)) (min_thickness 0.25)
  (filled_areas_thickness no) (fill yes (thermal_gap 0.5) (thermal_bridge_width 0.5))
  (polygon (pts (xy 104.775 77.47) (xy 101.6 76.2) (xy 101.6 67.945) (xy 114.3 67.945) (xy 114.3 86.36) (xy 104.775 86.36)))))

